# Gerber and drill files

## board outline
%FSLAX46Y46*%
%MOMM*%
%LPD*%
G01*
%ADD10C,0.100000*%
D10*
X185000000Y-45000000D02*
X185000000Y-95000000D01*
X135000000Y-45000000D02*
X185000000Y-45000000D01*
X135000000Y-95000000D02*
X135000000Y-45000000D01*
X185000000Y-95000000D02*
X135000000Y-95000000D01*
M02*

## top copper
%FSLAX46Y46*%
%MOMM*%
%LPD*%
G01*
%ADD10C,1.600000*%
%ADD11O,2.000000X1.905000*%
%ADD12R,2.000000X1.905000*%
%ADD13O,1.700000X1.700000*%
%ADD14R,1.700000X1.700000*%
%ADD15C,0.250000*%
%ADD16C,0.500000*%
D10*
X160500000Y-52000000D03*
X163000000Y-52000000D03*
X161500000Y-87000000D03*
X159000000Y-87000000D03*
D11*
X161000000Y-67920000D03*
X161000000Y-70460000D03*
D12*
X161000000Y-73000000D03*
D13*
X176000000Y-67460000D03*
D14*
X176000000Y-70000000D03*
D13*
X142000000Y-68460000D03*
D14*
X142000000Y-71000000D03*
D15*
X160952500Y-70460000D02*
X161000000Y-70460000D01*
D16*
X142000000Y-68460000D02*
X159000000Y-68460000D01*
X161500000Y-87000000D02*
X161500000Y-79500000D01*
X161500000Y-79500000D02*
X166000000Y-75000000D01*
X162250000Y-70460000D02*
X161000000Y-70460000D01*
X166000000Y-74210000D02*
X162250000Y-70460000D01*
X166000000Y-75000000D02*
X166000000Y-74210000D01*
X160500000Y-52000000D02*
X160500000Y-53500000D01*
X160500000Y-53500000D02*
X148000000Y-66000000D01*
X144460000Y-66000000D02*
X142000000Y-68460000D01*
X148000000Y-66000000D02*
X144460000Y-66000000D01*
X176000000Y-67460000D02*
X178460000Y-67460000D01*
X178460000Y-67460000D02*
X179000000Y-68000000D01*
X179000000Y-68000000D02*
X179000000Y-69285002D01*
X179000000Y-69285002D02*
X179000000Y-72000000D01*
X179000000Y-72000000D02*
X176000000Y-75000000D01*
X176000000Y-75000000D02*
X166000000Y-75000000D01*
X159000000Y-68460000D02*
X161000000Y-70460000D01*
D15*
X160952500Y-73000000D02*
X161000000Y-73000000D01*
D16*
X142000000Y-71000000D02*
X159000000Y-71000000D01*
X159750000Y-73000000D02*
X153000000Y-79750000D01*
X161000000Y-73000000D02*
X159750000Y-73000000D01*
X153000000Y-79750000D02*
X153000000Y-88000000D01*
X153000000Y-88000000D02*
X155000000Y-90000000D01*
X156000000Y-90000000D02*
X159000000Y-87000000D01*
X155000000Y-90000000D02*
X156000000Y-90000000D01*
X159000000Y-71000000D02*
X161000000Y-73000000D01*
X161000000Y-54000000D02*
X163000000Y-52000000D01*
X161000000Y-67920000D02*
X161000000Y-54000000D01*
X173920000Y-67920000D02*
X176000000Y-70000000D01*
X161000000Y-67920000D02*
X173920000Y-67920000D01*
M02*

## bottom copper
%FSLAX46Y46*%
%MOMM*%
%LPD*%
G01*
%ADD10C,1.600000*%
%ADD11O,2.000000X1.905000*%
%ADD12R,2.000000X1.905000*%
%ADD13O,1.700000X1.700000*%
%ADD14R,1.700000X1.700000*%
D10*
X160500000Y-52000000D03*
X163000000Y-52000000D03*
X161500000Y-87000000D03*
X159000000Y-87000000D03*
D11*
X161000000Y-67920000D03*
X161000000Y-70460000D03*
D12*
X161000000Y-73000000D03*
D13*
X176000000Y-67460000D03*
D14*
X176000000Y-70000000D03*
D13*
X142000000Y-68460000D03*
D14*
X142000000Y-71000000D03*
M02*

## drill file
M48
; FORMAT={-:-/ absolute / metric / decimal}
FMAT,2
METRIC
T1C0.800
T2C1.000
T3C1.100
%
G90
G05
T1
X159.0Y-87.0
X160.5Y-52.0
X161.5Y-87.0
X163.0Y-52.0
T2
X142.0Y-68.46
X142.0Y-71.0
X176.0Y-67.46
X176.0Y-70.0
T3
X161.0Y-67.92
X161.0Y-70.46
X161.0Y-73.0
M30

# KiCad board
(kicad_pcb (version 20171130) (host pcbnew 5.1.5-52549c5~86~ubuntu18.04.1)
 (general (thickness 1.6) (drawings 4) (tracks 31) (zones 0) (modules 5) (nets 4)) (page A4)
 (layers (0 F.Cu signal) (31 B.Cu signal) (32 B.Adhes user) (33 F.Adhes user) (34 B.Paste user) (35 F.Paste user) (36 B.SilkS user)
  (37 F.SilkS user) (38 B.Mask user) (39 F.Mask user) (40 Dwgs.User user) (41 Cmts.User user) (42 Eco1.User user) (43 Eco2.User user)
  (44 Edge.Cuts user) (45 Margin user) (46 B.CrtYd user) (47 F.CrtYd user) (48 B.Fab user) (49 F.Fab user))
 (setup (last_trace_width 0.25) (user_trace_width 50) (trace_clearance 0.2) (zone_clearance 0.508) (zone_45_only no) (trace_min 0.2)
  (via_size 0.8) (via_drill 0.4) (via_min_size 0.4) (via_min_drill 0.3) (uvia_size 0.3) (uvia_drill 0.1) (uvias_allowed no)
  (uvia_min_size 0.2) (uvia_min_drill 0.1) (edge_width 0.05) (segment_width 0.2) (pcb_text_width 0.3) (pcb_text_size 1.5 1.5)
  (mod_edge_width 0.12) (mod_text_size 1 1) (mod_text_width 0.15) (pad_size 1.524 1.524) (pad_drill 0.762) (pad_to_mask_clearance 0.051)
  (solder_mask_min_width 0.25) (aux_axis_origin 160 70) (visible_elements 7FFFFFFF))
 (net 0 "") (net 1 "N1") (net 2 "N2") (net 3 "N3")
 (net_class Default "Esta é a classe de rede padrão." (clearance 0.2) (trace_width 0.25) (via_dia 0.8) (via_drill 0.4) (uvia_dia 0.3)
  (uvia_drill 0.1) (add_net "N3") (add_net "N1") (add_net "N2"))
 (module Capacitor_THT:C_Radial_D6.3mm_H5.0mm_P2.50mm (layer F.Cu) (at 163 52 180)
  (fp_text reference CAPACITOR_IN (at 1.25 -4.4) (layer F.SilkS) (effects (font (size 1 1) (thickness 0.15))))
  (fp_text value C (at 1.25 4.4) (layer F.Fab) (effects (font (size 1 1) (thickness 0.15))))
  (pad 2 thru_hole circle (at 2.5 0 180) (size 1.6 1.6) (drill 0.8) (layers *.Cu *.Mask) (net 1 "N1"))
  (pad 1 thru_hole circle (at 0 0 180) (size 1.6 1.6) (drill 0.8) (layers *.Cu *.Mask) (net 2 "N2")))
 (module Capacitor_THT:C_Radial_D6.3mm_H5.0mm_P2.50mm (layer F.Cu) (at 159 87)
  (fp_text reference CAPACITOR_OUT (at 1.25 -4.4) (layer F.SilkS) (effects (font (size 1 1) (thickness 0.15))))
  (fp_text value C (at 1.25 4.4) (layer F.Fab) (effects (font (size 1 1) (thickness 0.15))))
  (pad 2 thru_hole circle (at 2.5 0) (size 1.6 1.6) (drill 0.8) (layers *.Cu *.Mask) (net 1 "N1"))
  (pad 1 thru_hole circle (at 0 0) (size 1.6 1.6) (drill 0.8) (layers *.Cu *.Mask) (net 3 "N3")))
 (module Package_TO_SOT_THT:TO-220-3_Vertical (layer F.Cu) (at 161 73 90)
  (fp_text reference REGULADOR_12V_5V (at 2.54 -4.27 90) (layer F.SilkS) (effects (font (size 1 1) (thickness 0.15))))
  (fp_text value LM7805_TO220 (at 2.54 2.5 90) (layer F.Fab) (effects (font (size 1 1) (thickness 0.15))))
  (pad 3 thru_hole oval (at 5.08 0 90) (size 1.905 2) (drill 1.1) (layers *.Cu *.Mask) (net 2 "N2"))
  (pad 2 thru_hole oval (at 2.54 0 90) (size 1.905 2) (drill 1.1) (layers *.Cu *.Mask) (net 1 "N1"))
  (pad 1 thru_hole rect (at 0 0 90) (size 1.905 2) (drill 1.1) (layers *.Cu *.Mask) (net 3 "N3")))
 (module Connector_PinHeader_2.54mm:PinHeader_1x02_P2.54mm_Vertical (layer F.Cu) (at 176 70 180)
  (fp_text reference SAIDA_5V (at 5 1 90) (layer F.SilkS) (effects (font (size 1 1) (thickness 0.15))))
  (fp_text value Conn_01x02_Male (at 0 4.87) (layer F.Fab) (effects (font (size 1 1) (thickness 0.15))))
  (pad 2 thru_hole oval (at 0 2.54 180) (size 1.7 1.7) (drill 1) (layers *.Cu *.Mask) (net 1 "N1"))
  (pad 1 thru_hole rect (at 0 0 180) (size 1.7 1.7) (drill 1) (layers *.Cu *.Mask) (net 2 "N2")))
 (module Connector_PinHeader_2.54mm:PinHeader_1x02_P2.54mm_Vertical (layer F.Cu) (at 142 71 180)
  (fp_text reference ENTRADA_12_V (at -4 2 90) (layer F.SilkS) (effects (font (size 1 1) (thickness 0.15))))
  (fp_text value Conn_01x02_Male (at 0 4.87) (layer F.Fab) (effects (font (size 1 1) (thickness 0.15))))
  (pad 2 thru_hole oval (at 0 2.54 180) (size 1.7 1.7) (drill 1) (layers *.Cu *.Mask) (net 1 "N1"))
  (pad 1 thru_hole rect (at 0 0 180) (size 1.7 1.7) (drill 1) (layers *.Cu *.Mask) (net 3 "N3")))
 (gr_line (start 185 45) (end 185 95) (layer Edge.Cuts) (width 0.1))
 (gr_line (start 135 45) (end 185 45) (layer Edge.Cuts) (width 0.1))
 (gr_line (start 135 95) (end 135 45) (layer Edge.Cuts) (width 0.1))
 (gr_line (start 185 95) (end 135 95) (layer Edge.Cuts) (width 0.1))
 (segment (start 160.9525 70.46) (end 161 70.46) (width 0.25) (layer F.Cu) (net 1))
 (segment (start 142 68.46) (end 159 68.46) (width 0.5) (layer F.Cu) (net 1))
 (segment (start 161.5 87) (end 161.5 79.5) (width 0.5) (layer F.Cu) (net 1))
 (segment (start 161.5 79.5) (end 166 75) (width 0.5) (layer F.Cu) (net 1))
 (segment (start 162.25 70.46) (end 161 70.46) (width 0.5) (layer F.Cu) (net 1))
 (segment (start 166 74.21) (end 162.25 70.46) (width 0.5) (layer F.Cu) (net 1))
 (segment (start 166 75) (end 166 74.21) (width 0.5) (layer F.Cu) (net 1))
 (segment (start 160.5 52) (end 160.5 53.5) (width 0.5) (layer F.Cu) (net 1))
 (segment (start 160.5 53.5) (end 148 66) (width 0.5) (layer F.Cu) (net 1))
 (segment (start 144.46 66) (end 142 68.46) (width 0.5) (layer F.Cu) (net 1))
 (segment (start 148 66) (end 144.46 66) (width 0.5) (layer F.Cu) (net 1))
 (segment (start 176 67.46) (end 178.46 67.46) (width 0.5) (layer F.Cu) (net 1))
 (segment (start 178.46 67.46) (end 179 68) (width 0.5) (layer F.Cu) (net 1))
 (segment (start 179 68) (end 179 69.285002) (width 0.5) (layer F.Cu) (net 1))
 (segment (start 179 69.285002) (end 179 72) (width 0.5) (layer F.Cu) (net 1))
 (segment (start 179 72) (end 176 75) (width 0.5) (layer F.Cu) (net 1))
 (segment (start 176 75) (end 166 75) (width 0.5) (layer F.Cu) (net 1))
 (segment (start 159 68.46) (end 161 70.46) (width 0.5) (layer F.Cu) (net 1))
 (segment (start 160.9525 73) (end 161 73) (width 0.25) (layer F.Cu) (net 3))
 (segment (start 142 71) (end 159 71) (width 0.5) (layer F.Cu) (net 3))
 (segment (start 159.75 73) (end 153 79.75) (width 0.5) (layer F.Cu) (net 3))
 (segment (start 161 73) (end 159.75 73) (width 0.5) (layer F.Cu) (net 3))
 (segment (start 153 79.75) (end 153 88) (width 0.5) (layer F.Cu) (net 3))
 (segment (start 153 88) (end 155 90) (width 0.5) (layer F.Cu) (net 3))
 (segment (start 156 90) (end 159 87) (width 0.5) (layer F.Cu) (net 3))
 (segment (start 155 90) (end 156 90) (width 0.5) (layer F.Cu) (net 3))
 (segment (start 159 71) (end 161 73) (width 0.5) (layer F.Cu) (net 3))
 (segment (start 161 54) (end 163 52) (width 0.5) (layer F.Cu) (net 2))
 (segment (start 161 67.92) (end 161 54) (width 0.5) (layer F.Cu) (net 2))
 (segment (start 173.92 67.92) (end 176 70) (width 0.5) (layer F.Cu) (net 2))
 (segment (start 161 67.92) (end 173.92 67.92) (width 0.5) (layer F.Cu) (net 2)))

